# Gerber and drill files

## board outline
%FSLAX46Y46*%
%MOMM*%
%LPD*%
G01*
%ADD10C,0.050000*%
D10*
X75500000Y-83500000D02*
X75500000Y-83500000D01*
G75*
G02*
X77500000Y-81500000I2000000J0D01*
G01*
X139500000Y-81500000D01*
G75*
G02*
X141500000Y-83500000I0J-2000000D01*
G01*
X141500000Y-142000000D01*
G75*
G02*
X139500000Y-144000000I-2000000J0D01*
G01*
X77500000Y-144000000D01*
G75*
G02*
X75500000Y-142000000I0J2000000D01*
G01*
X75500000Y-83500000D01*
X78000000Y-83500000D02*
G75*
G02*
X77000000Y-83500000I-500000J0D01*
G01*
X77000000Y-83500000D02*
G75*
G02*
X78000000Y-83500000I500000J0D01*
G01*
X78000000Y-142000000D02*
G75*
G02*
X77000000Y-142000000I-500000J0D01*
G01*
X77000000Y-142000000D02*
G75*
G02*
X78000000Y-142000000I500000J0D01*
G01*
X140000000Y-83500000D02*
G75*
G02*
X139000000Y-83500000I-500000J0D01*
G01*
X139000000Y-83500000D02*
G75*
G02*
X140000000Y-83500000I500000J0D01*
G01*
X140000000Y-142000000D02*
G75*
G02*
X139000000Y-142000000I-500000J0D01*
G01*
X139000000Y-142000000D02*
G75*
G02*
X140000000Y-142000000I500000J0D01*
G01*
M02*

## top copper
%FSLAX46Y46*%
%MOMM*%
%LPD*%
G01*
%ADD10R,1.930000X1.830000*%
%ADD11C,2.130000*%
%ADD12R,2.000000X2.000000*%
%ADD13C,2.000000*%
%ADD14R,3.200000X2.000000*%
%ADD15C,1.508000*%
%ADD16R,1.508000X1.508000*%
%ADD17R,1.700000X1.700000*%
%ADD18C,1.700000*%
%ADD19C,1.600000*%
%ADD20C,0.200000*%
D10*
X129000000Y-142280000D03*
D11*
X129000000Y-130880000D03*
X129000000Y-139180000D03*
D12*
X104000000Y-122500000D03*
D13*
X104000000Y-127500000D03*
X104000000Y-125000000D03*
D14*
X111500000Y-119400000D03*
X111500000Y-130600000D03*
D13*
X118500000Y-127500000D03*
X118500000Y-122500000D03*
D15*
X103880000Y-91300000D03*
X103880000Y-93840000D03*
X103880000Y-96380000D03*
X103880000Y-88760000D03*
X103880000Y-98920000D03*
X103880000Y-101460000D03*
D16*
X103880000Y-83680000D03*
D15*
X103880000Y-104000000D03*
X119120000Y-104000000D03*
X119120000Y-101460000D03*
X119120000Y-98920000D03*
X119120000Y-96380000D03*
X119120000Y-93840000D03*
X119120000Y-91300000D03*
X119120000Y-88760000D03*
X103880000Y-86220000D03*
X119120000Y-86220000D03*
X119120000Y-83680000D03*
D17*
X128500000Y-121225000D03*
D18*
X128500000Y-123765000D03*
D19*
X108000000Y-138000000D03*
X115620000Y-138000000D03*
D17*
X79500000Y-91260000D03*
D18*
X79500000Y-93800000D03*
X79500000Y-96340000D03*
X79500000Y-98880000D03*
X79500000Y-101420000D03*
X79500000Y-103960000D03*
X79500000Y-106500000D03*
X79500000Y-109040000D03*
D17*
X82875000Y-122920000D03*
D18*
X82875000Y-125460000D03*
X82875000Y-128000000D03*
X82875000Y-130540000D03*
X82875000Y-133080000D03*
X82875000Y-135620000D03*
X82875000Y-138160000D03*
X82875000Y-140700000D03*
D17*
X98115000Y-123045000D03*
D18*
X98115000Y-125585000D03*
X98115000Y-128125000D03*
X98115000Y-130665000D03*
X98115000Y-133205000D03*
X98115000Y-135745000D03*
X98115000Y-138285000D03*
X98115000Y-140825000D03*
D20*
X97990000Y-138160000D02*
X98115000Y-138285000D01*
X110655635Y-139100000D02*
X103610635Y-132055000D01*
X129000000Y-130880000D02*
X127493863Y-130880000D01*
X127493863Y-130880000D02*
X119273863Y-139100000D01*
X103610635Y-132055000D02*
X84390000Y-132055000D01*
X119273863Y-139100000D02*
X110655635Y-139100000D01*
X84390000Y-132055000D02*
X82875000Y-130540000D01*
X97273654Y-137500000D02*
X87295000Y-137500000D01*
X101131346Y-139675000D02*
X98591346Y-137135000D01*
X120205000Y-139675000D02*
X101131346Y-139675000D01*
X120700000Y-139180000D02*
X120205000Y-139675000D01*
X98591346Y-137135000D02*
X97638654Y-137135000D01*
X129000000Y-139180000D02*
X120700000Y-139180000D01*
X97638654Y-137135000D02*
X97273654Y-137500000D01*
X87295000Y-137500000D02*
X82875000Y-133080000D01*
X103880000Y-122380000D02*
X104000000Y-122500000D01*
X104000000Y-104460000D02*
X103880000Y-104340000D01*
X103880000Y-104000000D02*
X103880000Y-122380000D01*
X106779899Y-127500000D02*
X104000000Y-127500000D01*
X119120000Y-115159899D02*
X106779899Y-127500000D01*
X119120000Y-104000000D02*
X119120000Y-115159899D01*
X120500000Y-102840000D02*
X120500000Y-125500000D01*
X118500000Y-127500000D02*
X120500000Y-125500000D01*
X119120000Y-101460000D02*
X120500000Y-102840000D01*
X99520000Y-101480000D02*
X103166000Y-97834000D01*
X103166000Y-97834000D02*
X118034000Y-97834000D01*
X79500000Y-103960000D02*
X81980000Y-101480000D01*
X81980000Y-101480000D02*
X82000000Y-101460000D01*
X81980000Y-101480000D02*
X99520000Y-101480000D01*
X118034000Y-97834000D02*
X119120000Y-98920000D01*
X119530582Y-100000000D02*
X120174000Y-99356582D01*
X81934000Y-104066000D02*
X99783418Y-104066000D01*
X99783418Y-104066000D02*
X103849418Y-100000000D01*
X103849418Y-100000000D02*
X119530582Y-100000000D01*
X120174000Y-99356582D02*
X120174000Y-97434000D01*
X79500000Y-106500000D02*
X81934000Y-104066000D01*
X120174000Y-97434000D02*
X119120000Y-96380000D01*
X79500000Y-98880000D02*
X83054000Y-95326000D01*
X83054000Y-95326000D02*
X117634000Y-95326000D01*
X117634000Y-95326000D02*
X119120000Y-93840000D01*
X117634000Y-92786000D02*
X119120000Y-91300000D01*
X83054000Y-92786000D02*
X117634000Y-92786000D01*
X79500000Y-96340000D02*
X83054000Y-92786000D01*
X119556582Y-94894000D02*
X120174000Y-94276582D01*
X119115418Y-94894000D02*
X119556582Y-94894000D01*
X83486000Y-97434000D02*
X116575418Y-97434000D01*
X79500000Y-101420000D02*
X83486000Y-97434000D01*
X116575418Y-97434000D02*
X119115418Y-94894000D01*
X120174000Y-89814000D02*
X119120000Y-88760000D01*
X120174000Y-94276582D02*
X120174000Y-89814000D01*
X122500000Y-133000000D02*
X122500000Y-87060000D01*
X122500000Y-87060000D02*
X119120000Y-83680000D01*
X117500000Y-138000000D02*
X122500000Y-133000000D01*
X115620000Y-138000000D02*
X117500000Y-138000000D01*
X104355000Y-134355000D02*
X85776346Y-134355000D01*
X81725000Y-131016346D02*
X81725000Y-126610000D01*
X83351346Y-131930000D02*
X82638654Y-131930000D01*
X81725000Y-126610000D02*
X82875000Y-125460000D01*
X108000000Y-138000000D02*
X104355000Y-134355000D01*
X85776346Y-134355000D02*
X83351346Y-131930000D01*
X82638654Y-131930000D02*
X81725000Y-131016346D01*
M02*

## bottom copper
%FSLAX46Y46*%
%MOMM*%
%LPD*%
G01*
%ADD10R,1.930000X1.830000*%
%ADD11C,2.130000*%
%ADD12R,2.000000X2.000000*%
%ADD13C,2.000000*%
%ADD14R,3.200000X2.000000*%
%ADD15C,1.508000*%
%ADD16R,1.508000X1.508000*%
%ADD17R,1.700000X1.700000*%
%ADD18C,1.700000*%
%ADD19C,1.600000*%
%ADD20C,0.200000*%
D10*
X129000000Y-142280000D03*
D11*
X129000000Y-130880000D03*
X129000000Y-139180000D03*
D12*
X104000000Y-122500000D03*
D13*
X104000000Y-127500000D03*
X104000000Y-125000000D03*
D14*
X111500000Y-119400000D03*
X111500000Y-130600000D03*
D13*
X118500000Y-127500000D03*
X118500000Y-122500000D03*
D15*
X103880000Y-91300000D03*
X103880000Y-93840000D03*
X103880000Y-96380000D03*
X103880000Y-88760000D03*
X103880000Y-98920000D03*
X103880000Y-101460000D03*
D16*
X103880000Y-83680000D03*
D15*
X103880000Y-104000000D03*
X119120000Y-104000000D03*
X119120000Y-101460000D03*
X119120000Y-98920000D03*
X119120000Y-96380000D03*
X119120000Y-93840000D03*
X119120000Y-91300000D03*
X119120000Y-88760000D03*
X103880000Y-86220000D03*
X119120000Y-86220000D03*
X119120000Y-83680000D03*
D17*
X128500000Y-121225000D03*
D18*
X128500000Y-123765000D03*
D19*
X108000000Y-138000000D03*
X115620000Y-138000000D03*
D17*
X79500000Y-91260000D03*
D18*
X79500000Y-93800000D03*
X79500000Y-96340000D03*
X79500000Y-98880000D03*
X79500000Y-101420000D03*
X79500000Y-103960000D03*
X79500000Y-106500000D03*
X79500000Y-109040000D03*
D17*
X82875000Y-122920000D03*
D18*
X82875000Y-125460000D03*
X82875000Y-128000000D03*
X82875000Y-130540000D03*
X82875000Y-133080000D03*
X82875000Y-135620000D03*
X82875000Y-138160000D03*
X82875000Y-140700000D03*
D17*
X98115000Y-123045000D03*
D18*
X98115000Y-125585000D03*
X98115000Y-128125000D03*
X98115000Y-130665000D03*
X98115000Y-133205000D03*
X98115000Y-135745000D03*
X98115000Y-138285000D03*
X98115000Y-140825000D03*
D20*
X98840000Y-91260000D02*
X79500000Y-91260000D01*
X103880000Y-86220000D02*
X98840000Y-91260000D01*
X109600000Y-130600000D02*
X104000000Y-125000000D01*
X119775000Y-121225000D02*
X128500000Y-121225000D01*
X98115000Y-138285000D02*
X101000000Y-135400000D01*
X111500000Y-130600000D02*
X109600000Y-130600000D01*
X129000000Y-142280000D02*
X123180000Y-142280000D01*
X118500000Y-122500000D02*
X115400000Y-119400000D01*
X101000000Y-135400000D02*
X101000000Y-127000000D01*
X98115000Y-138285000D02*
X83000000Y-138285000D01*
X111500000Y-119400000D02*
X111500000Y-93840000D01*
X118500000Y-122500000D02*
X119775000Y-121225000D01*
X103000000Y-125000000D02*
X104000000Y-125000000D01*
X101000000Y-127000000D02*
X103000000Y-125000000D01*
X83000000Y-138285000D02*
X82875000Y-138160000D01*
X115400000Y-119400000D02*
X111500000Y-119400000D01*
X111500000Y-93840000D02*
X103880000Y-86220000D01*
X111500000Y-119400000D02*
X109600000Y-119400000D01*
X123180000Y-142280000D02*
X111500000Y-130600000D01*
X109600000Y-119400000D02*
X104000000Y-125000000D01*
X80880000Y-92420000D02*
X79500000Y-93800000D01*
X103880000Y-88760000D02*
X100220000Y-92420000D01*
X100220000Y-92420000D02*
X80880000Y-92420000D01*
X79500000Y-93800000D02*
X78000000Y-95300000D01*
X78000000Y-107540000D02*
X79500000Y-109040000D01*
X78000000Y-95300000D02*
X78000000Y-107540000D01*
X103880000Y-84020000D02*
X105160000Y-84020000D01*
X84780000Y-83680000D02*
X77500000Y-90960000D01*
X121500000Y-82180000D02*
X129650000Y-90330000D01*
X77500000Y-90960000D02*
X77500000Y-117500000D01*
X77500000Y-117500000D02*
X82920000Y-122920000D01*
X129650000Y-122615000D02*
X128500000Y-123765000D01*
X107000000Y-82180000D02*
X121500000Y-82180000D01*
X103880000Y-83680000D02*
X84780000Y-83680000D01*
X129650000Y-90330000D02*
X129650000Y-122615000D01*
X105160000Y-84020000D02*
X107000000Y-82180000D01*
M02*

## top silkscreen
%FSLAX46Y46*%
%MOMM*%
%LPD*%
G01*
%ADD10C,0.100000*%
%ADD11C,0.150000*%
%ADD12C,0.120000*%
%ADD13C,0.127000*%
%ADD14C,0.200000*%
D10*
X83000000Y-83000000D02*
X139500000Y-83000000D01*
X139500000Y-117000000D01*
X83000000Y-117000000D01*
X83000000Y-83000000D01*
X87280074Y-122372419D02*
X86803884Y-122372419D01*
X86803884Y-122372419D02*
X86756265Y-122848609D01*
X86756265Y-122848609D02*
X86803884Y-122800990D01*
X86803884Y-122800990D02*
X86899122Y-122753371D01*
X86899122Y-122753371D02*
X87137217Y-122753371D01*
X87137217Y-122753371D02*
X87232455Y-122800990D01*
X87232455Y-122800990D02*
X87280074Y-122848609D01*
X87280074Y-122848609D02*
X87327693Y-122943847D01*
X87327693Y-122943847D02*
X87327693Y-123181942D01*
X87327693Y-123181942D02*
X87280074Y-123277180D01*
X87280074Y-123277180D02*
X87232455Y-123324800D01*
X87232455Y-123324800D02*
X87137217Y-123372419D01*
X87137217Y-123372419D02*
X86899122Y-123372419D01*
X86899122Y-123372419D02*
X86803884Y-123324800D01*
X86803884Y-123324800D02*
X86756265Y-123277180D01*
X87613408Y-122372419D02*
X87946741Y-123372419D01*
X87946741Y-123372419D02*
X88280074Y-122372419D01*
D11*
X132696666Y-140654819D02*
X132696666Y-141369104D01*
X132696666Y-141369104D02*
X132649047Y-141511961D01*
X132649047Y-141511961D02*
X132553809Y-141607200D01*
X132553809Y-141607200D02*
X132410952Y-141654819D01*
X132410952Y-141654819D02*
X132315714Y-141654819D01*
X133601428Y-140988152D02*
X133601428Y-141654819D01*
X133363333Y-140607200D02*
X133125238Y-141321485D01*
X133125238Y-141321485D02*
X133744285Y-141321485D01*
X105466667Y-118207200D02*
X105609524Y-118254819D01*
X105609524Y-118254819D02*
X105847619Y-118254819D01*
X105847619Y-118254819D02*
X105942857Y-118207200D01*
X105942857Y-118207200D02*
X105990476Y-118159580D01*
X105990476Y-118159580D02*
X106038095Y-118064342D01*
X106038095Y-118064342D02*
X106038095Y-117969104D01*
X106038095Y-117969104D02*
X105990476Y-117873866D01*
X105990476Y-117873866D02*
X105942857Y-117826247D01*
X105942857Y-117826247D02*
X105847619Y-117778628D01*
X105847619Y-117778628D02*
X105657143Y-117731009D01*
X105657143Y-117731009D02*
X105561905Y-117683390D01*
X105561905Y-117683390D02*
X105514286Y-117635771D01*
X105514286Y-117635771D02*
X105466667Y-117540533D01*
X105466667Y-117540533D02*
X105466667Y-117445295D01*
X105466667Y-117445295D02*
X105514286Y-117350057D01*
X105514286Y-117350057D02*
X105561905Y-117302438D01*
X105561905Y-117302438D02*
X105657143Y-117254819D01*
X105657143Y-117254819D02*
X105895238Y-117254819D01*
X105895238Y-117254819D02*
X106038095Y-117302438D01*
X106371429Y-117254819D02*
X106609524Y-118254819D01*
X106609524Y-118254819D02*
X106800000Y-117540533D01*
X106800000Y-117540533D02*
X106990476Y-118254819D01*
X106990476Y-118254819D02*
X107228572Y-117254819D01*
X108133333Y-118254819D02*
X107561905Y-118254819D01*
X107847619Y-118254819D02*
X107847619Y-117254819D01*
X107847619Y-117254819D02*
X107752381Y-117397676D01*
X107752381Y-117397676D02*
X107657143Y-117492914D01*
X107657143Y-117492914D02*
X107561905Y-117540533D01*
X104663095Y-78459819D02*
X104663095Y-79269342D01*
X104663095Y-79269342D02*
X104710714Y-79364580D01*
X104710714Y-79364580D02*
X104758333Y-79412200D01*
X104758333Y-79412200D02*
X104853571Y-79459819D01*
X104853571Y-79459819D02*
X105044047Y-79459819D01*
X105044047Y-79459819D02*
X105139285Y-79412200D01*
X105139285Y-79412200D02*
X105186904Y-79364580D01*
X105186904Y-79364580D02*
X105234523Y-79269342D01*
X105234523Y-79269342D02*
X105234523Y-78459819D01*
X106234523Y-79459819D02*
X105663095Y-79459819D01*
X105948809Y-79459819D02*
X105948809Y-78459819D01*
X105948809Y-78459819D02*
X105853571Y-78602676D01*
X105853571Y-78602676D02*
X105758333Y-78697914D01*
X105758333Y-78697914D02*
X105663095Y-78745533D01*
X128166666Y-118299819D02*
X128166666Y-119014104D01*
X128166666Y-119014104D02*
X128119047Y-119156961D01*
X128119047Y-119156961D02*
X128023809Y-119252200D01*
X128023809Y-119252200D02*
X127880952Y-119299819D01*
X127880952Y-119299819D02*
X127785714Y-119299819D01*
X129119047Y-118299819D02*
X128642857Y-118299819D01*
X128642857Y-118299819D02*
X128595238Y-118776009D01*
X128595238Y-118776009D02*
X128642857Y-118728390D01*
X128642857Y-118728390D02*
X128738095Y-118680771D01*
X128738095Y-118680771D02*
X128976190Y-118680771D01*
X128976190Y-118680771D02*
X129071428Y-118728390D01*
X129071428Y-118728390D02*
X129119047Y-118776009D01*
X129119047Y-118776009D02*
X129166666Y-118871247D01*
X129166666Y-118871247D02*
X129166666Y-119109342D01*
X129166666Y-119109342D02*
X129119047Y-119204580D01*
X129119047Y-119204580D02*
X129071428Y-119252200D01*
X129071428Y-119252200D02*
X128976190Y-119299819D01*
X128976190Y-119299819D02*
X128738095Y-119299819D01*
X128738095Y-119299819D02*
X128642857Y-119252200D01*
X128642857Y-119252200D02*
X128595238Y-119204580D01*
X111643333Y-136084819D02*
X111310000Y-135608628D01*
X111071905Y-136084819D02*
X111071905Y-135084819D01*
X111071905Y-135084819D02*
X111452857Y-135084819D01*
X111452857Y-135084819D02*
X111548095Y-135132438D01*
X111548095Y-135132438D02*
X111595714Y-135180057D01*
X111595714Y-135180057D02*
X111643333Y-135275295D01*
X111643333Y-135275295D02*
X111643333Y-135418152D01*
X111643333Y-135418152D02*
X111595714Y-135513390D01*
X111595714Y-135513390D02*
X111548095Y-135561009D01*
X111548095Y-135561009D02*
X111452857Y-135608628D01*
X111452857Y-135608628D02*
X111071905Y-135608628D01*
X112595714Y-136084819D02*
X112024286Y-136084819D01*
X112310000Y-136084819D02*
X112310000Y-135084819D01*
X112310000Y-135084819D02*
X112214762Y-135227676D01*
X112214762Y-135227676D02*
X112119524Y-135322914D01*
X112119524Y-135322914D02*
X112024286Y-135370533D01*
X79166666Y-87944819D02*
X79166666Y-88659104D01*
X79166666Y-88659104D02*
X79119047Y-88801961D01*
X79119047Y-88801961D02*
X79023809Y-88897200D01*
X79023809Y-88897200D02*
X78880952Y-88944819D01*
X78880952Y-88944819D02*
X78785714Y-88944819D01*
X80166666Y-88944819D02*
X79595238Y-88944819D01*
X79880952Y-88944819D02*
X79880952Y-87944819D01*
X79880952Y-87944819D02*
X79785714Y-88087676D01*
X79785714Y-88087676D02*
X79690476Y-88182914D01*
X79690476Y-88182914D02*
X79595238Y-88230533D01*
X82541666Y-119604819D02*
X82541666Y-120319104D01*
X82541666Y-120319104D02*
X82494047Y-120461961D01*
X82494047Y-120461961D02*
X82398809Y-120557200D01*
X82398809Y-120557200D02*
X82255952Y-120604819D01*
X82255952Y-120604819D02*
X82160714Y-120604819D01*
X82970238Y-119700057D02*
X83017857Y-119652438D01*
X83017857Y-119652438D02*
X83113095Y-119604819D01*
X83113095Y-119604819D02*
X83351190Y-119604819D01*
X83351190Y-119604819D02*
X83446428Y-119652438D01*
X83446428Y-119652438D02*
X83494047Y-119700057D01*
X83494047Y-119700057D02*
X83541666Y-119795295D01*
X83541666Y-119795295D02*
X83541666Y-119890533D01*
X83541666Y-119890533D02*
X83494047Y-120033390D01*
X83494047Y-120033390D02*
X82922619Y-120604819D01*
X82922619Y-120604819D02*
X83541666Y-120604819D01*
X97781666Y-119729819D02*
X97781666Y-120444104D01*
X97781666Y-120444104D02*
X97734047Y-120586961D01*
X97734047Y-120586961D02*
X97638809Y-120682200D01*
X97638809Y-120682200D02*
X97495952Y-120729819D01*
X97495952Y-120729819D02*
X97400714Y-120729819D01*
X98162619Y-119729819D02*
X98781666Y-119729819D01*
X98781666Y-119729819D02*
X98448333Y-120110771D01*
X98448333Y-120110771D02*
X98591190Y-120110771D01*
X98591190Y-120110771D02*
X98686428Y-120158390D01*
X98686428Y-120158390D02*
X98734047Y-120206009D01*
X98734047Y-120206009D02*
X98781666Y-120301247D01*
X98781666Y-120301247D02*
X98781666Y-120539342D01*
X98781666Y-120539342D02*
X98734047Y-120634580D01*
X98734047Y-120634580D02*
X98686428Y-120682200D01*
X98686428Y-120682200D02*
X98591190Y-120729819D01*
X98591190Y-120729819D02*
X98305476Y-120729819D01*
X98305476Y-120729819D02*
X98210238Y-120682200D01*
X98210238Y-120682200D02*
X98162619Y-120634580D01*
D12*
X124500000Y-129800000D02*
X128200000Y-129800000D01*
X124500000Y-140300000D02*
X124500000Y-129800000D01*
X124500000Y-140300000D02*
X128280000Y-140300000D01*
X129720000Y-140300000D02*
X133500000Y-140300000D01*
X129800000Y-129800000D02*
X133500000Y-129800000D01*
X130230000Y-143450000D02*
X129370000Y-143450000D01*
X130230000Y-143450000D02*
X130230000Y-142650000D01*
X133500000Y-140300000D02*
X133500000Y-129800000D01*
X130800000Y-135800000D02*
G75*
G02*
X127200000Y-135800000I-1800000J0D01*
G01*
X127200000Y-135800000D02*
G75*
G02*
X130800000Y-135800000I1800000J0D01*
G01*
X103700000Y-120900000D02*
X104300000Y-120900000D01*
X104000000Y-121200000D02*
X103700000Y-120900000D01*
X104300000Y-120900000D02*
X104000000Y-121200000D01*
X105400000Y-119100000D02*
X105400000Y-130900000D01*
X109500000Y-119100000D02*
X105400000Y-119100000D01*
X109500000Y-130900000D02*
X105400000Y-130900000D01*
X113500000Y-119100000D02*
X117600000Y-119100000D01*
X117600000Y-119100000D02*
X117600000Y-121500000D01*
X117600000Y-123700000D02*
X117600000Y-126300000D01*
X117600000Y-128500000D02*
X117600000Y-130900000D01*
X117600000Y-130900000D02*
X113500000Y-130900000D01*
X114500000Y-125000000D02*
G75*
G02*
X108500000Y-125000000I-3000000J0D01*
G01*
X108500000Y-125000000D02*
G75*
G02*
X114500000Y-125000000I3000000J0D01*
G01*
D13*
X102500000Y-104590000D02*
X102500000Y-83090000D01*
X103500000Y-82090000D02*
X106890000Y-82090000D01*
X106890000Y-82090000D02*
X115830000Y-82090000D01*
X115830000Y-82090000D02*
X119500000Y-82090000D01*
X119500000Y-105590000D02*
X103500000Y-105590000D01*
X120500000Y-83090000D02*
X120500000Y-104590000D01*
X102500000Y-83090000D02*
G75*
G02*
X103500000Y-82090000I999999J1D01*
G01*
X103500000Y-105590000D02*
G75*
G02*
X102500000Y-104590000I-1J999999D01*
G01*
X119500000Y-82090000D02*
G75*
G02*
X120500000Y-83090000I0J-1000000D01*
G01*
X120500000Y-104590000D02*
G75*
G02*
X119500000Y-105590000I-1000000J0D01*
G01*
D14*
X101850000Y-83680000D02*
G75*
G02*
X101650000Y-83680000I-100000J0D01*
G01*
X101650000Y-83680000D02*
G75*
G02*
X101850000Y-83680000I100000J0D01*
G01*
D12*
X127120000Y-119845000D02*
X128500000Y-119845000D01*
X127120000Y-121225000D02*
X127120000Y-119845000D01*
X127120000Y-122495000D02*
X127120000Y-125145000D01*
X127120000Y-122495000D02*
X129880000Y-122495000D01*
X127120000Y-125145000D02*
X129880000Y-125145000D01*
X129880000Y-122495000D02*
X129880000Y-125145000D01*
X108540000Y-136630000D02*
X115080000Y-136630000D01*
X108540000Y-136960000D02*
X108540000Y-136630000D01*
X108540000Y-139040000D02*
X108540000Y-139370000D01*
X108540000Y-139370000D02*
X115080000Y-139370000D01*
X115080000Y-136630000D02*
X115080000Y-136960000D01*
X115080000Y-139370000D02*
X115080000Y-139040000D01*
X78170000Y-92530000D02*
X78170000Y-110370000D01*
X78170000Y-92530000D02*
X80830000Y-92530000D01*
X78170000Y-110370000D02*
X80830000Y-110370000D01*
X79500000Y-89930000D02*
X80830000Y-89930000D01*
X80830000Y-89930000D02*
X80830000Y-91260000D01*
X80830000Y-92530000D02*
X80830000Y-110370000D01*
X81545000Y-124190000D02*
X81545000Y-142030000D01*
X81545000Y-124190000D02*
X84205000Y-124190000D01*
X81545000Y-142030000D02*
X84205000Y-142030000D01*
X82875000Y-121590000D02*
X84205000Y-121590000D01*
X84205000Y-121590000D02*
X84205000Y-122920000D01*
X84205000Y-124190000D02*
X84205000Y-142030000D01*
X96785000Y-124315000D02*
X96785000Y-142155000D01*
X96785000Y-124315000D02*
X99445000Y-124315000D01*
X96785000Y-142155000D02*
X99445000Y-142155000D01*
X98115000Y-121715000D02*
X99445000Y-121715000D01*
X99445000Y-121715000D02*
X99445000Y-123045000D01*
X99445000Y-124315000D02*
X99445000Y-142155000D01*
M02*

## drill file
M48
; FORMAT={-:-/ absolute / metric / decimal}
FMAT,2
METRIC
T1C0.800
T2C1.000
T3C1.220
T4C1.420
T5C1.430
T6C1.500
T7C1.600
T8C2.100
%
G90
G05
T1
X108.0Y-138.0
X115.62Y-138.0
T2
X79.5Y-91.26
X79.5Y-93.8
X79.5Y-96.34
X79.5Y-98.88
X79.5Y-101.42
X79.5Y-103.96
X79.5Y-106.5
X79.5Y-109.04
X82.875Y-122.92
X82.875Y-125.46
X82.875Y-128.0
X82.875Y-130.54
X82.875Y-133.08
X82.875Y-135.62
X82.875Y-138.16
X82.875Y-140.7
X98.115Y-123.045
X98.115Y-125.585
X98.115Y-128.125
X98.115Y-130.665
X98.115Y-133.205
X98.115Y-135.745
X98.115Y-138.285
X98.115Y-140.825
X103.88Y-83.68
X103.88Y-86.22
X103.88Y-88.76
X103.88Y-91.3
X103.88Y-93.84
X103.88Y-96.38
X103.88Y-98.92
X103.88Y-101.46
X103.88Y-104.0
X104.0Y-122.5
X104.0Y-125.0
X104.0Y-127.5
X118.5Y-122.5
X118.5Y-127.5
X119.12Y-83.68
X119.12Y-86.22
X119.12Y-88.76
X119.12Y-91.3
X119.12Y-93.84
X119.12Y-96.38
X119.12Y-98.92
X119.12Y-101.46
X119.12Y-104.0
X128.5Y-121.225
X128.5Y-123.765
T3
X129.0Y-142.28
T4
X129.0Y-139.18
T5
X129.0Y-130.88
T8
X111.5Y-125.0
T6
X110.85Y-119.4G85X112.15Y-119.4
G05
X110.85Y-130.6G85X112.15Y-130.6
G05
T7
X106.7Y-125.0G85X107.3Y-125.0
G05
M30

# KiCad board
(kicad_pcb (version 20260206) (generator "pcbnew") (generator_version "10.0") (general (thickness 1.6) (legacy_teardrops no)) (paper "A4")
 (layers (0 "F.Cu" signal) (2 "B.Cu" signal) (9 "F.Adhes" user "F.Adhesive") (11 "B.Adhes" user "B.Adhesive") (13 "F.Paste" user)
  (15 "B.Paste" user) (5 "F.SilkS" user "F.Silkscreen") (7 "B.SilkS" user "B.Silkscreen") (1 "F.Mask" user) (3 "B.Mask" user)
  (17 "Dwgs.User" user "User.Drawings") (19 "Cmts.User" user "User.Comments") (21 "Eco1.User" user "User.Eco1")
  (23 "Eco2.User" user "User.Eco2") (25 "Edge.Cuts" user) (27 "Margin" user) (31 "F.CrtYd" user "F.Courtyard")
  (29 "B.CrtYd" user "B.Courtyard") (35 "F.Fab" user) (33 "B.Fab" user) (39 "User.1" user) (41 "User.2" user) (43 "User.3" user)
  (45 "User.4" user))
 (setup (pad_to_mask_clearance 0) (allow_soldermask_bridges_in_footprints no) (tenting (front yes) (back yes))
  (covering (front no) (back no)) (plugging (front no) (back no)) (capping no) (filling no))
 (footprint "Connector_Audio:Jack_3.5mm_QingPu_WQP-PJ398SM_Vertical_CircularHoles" (layer "F.Cu") (at 129 142.28 180)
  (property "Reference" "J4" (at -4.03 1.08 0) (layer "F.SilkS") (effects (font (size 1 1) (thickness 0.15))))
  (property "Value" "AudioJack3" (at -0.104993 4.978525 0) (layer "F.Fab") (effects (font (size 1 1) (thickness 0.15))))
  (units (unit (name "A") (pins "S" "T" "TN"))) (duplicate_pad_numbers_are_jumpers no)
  (fp_line (start 4.5 12.48) (end 0.8 12.48) (stroke (width 0.12) (type solid)) (layer "F.SilkS"))
  (fp_line (start 4.5 1.98) (end 4.5 12.48) (stroke (width 0.12) (type solid)) (layer "F.SilkS"))
  (fp_line (start 4.5 1.98) (end 0.72 1.98) (stroke (width 0.12) (type solid)) (layer "F.SilkS"))
  (fp_line (start -0.72 1.98) (end -4.5 1.98) (stroke (width 0.12) (type solid)) (layer "F.SilkS"))
  (fp_line (start -0.8 12.48) (end -4.5 12.48) (stroke (width 0.12) (type solid)) (layer "F.SilkS"))
  (fp_line (start -1.23 -1.17) (end -0.37 -1.17) (stroke (width 0.12) (type solid)) (layer "F.SilkS"))
  (fp_line (start -1.23 -1.17) (end -1.23 -0.37) (stroke (width 0.12) (type solid)) (layer "F.SilkS"))
  (fp_line (start -4.5 1.98) (end -4.5 12.48) (stroke (width 0.12) (type solid)) (layer "F.SilkS"))
  (fp_circle (center 0 6.48) (end 1.8 6.48) (stroke (width 0.12) (type solid)) (fill no) (layer "F.SilkS"))
  (pad "S" thru_hole rect (at 0 0) (size 1.93 1.83) (drill 1.22) (layers "*.Cu" "*.Mask") (remove_unused_layers no) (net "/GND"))
  (pad "T" thru_hole circle (at 0 11.4) (size 2.13 2.13) (drill 1.43) (layers "*.Cu" "*.Mask") (remove_unused_layers no) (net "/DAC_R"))
  (pad "TN" thru_hole circle (at 0 3.1) (size 2.13 2.13) (drill 1.42) (layers "*.Cu" "*.Mask") (remove_unused_layers no) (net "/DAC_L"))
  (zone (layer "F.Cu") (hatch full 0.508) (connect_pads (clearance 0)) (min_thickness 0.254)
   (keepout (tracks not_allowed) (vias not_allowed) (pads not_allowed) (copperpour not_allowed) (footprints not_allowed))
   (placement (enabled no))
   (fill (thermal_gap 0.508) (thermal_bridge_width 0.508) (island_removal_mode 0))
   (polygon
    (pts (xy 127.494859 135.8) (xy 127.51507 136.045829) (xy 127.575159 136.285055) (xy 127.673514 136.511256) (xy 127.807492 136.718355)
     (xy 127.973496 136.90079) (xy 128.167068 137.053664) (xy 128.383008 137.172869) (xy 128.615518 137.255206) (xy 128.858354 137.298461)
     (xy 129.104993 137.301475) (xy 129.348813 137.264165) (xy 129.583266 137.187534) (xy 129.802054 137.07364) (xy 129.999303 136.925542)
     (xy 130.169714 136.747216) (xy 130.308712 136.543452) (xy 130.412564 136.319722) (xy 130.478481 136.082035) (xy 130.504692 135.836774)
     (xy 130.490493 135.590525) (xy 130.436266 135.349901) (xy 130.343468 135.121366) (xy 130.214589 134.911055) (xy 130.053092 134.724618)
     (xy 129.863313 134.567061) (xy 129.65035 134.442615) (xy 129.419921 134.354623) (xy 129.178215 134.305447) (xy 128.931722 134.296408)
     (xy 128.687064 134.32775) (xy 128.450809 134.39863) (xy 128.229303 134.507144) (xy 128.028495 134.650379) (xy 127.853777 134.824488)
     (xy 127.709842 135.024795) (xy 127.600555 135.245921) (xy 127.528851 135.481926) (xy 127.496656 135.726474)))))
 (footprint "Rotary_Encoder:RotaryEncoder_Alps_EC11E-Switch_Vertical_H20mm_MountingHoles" (layer "F.Cu") (at 104 122.5)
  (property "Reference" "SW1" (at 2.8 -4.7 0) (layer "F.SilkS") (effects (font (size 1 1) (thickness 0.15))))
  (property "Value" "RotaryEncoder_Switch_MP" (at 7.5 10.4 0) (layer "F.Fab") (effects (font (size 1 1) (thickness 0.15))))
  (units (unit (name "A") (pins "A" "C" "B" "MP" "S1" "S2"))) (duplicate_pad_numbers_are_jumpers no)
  (fp_line (start -0.3 -1.6) (end 0.3 -1.6) (stroke (width 0.12) (type solid)) (layer "F.SilkS"))
  (fp_line (start 0 -1.3) (end -0.3 -1.6) (stroke (width 0.12) (type solid)) (layer "F.SilkS"))
  (fp_line (start 0.3 -1.6) (end 0 -1.3) (stroke (width 0.12) (type solid)) (layer "F.SilkS"))
  (fp_line (start 1.4 -3.4) (end 1.4 8.4) (stroke (width 0.12) (type solid)) (layer "F.SilkS"))
  (fp_line (start 5.5 -3.4) (end 1.4 -3.4) (stroke (width 0.12) (type solid)) (layer "F.SilkS"))
  (fp_line (start 5.5 8.4) (end 1.4 8.4) (stroke (width 0.12) (type solid)) (layer "F.SilkS"))
  (fp_line (start 9.5 -3.4) (end 13.6 -3.4) (stroke (width 0.12) (type solid)) (layer "F.SilkS"))
  (fp_line (start 13.6 -3.4) (end 13.6 -1) (stroke (width 0.12) (type solid)) (layer "F.SilkS"))
  (fp_line (start 13.6 1.2) (end 13.6 3.8) (stroke (width 0.12) (type solid)) (layer "F.SilkS"))
  (fp_line (start 13.6 6) (end 13.6 8.4) (stroke (width 0.12) (type solid)) (layer "F.SilkS"))
  (fp_line (start 13.6 8.4) (end 9.5 8.4) (stroke (width 0.12) (type solid)) (layer "F.SilkS"))
  (fp_circle (center 7.5 2.5) (end 10.5 2.5) (stroke (width 0.12) (type solid)) (fill no) (layer "F.SilkS"))
  (pad "" np_thru_hole oval (at 3 2.5) (size 2.2 1.6) (drill oval 2.2 1.6) (layers "*.Mask"))
  (pad "" np_thru_hole circle (at 7.5 2.5) (size 2.1 2.1) (drill 2.1) (layers "*.Mask"))
  (pad "A" thru_hole rect (at 0 0) (size 2 2) (drill 1) (layers "*.Cu" "*.Mask") (remove_unused_layers no) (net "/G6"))
  (pad "B" thru_hole circle (at 0 5) (size 2 2) (drill 1) (layers "*.Cu" "*.Mask") (remove_unused_layers no) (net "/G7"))
  (pad "C" thru_hole circle (at 0 2.5) (size 2 2) (drill 1) (layers "*.Cu" "*.Mask") (remove_unused_layers no) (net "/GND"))
  (pad "MP" thru_hole rect (at 7.5 -3.1) (size 3.2 2) (drill oval 2.8 1.5) (layers "*.Cu" "*.Mask") (remove_unused_layers no) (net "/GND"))
  (pad "MP" thru_hole rect (at 7.5 8.1) (size 3.2 2) (drill oval 2.8 1.5) (layers "*.Cu" "*.Mask") (remove_unused_layers no) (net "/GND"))
  (pad "S1" thru_hole circle (at 14.5 5) (size 2 2) (drill 1) (layers "*.Cu" "*.Mask") (remove_unused_layers no) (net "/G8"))
  (pad "S2" thru_hole circle (at 14.5 0) (size 2 2) (drill 1) (layers "*.Cu" "*.Mask") (remove_unused_layers no) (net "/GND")))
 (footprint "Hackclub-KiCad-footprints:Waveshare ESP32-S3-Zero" (layer "F.Cu") (at 111.5 93.84)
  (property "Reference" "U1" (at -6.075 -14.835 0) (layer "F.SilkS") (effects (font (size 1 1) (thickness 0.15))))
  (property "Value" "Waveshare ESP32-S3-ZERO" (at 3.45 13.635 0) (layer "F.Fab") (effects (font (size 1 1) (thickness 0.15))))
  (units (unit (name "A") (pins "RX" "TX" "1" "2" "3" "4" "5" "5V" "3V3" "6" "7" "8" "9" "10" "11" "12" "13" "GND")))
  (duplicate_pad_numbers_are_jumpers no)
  (fp_line (start -9 10.75) (end -9 -10.75) (stroke (width 0.127) (type solid)) (layer "F.SilkS"))
  (fp_line (start -8 -11.75) (end -4.61 -11.75) (stroke (width 0.127) (type solid)) (layer "F.SilkS"))
  (fp_line (start -4.61 -11.75) (end 4.33 -11.75) (stroke (width 0.127) (type solid)) (layer "F.SilkS"))
  (fp_line (start 4.33 -11.75) (end 8 -11.75) (stroke (width 0.127) (type solid)) (layer "F.SilkS"))
  (fp_line (start 8 11.75) (end -8 11.75) (stroke (width 0.127) (type solid)) (layer "F.SilkS"))
  (fp_line (start 9 -10.75) (end 9 10.75) (stroke (width 0.127) (type solid)) (layer "F.SilkS"))
  (fp_arc (start -9 -10.75) (mid -8.707107 -11.457107) (end -8 -11.75) (stroke (width 0.127) (type solid)) (layer "F.SilkS"))
  (fp_arc (start -8 11.75) (mid -8.707107 11.457107) (end -9 10.75) (stroke (width 0.127) (type solid)) (layer "F.SilkS"))
  (fp_arc (start 8 -11.75) (mid 8.707107 -11.457107) (end 9 -10.75) (stroke (width 0.127) (type solid)) (layer "F.SilkS"))
  (fp_arc (start 9 10.75) (mid 8.707107 11.457107) (end 8 11.75) (stroke (width 0.127) (type solid)) (layer "F.SilkS"))
  (fp_circle (center -9.75 -10.16) (end -9.65 -10.16) (stroke (width 0.2) (type solid)) (fill no) (layer "F.SilkS"))
  (pad "1" thru_hole circle (at -7.62 -2.54) (size 1.508 1.508) (drill 1) (layers "*.Cu" "*.Mask") (remove_unused_layers no)
   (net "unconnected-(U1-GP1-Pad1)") (solder_mask_margin 0.102))
  (pad "2" thru_hole circle (at -7.62 0) (size 1.508 1.508) (drill 1) (layers "*.Cu" "*.Mask") (remove_unused_layers no)
   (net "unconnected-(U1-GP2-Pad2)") (solder_mask_margin 0.102))
  (pad "3" thru_hole circle (at -7.62 2.54) (size 1.508 1.508) (drill 1) (layers "*.Cu" "*.Mask") (remove_unused_layers no)
   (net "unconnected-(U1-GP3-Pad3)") (solder_mask_margin 0.102))
  (pad "3V3" thru_hole circle (at -7.62 -5.08) (size 1.508 1.508) (drill 1) (layers "*.Cu" "*.Mask") (remove_unused_layers no) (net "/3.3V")
   (solder_mask_margin 0.102))
  (pad "4" thru_hole circle (at -7.62 5.08) (size 1.508 1.508) (drill 1) (layers "*.Cu" "*.Mask") (remove_unused_layers no)
   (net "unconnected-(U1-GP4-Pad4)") (solder_mask_margin 0.102))
  (pad "5" thru_hole circle (at -7.62 7.62) (size 1.508 1.508) (drill 1) (layers "*.Cu" "*.Mask") (remove_unused_layers no)
   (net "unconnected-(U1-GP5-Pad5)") (solder_mask_margin 0.102))
  (pad "5V" thru_hole rect (at -7.62 -10.16) (size 1.508 1.508) (drill 1) (layers "*.Cu" "*.Mask") (remove_unused_layers no) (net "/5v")
   (solder_mask_margin 0.102))
  (pad "6" thru_hole circle (at -7.62 10.16) (size 1.508 1.508) (drill 1) (layers "*.Cu" "*.Mask") (remove_unused_layers no) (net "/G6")
   (solder_mask_margin 0.102))
  (pad "7" thru_hole circle (at 7.62 10.16) (size 1.508 1.508) (drill 1) (layers "*.Cu" "*.Mask") (remove_unused_layers no) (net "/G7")
   (solder_mask_margin 0.102))
  (pad "8" thru_hole circle (at 7.62 7.62) (size 1.508 1.508) (drill 1) (layers "*.Cu" "*.Mask") (remove_unused_layers no) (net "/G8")
   (solder_mask_margin 0.102))
  (pad "9" thru_hole circle (at 7.62 5.08) (size 1.508 1.508) (drill 1) (layers "*.Cu" "*.Mask") (remove_unused_layers no)
   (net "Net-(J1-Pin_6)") (solder_mask_margin 0.102))
  (pad "10" thru_hole circle (at 7.62 2.54) (size 1.508 1.508) (drill 1) (layers "*.Cu" "*.Mask") (remove_unused_layers no)
   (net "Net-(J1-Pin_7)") (solder_mask_margin 0.102))
  (pad "11" thru_hole circle (at 7.62 0) (size 1.508 1.508) (drill 1) (layers "*.Cu" "*.Mask") (remove_unused_layers no)
   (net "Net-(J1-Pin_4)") (solder_mask_margin 0.102))
  (pad "12" thru_hole circle (at 7.62 -2.54) (size 1.508 1.508) (drill 1) (layers "*.Cu" "*.Mask") (remove_unused_layers no)
   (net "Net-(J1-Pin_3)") (solder_mask_margin 0.102))
  (pad "13" thru_hole circle (at 7.62 -5.08) (size 1.508 1.508) (drill 1) (layers "*.Cu" "*.Mask") (remove_unused_layers no)
   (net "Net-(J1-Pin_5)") (solder_mask_margin 0.102))
  (pad "GND" thru_hole circle (at -7.62 -7.62) (size 1.508 1.508) (drill 1) (layers "*.Cu" "*.Mask") (remove_unused_layers no) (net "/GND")
   (solder_mask_margin 0.102))
  (pad "RX" thru_hole circle (at 7.62 -7.62) (size 1.508 1.508) (drill 1) (layers "*.Cu" "*.Mask") (remove_unused_layers no)
   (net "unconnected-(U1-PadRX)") (solder_mask_margin 0.102))
  (pad "TX" thru_hole circle (at 7.62 -10.16) (size 1.508 1.508) (drill 1) (layers "*.Cu" "*.Mask") (remove_unused_layers no)
   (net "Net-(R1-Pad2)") (solder_mask_margin 0.102)))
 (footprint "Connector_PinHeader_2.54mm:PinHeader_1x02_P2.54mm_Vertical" (layer "F.Cu") (at 128.5 121.225)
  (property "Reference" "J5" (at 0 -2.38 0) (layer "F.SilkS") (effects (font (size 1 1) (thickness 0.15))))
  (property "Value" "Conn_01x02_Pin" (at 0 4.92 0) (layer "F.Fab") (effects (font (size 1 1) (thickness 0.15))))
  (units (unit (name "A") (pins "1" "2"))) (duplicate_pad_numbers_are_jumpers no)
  (fp_line (start -1.38 -1.38) (end 0 -1.38) (stroke (width 0.12) (type solid)) (layer "F.SilkS"))
  (fp_line (start -1.38 0) (end -1.38 -1.38) (stroke (width 0.12) (type solid)) (layer "F.SilkS"))
  (fp_line (start -1.38 1.27) (end -1.38 3.92) (stroke (width 0.12) (type solid)) (layer "F.SilkS"))
  (fp_line (start -1.38 1.27) (end 1.38 1.27) (stroke (width 0.12) (type solid)) (layer "F.SilkS"))
  (fp_line (start -1.38 3.92) (end 1.38 3.92) (stroke (width 0.12) (type solid)) (layer "F.SilkS"))
  (fp_line (start 1.38 1.27) (end 1.38 3.92) (stroke (width 0.12) (type solid)) (layer "F.SilkS"))
  (pad "1" thru_hole rect (at 0 0) (size 1.7 1.7) (drill 1) (layers "*.Cu" "*.Mask") (remove_unused_layers no) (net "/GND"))
  (pad "2" thru_hole circle (at 0 2.54) (size 1.7 1.7) (drill 1) (layers "*.Cu" "*.Mask") (remove_unused_layers no) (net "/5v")))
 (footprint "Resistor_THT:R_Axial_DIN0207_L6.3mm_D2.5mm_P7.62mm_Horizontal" (layer "F.Cu") (at 108 138)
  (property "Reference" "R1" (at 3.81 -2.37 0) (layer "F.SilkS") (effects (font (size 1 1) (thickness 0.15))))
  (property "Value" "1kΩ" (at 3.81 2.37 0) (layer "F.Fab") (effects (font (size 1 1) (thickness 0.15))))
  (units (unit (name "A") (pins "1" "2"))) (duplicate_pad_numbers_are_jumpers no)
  (fp_line (start 0.54 -1.37) (end 7.08 -1.37) (stroke (width 0.12) (type solid)) (layer "F.SilkS"))
  (fp_line (start 0.54 -1.04) (end 0.54 -1.37) (stroke (width 0.12) (type solid)) (layer "F.SilkS"))
  (fp_line (start 0.54 1.04) (end 0.54 1.37) (stroke (width 0.12) (type solid)) (layer "F.SilkS"))
  (fp_line (start 0.54 1.37) (end 7.08 1.37) (stroke (width 0.12) (type solid)) (layer "F.SilkS"))
  (fp_line (start 7.08 -1.37) (end 7.08 -1.04) (stroke (width 0.12) (type solid)) (layer "F.SilkS"))
  (fp_line (start 7.08 1.37) (end 7.08 1.04) (stroke (width 0.12) (type solid)) (layer "F.SilkS"))
  (pad "1" thru_hole circle (at 0 0) (size 1.6 1.6) (drill 0.8) (layers "*.Cu" "*.Mask") (remove_unused_layers no) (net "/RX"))
  (pad "2" thru_hole circle (at 7.62 0) (size 1.6 1.6) (drill 0.8) (layers "*.Cu" "*.Mask") (remove_unused_layers no) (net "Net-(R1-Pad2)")))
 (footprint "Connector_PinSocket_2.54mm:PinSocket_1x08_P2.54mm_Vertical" (layer "F.Cu") (at 79.5 91.26)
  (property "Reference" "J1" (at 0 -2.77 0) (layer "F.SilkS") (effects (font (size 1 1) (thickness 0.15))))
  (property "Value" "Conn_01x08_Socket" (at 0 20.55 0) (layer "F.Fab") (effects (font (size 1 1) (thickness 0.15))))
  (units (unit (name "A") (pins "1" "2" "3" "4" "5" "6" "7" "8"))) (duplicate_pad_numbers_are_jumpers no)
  (fp_line (start -1.33 1.27) (end -1.33 19.11) (stroke (width 0.12) (type solid)) (layer "F.SilkS"))
  (fp_line (start -1.33 1.27) (end 1.33 1.27) (stroke (width 0.12) (type solid)) (layer "F.SilkS"))
  (fp_line (start -1.33 19.11) (end 1.33 19.11) (stroke (width 0.12) (type solid)) (layer "F.SilkS"))
  (fp_line (start 0 -1.33) (end 1.33 -1.33) (stroke (width 0.12) (type solid)) (layer "F.SilkS"))
  (fp_line (start 1.33 -1.33) (end 1.33 0) (stroke (width 0.12) (type solid)) (layer "F.SilkS"))
  (fp_line (start 1.33 1.27) (end 1.33 19.11) (stroke (width 0.12) (type solid)) (layer "F.SilkS"))
  (pad "1" thru_hole rect (at 0 0) (size 1.7 1.7) (drill 1) (layers "*.Cu" "*.Mask") (remove_unused_layers no) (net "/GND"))
  (pad "2" thru_hole circle (at 0 2.54) (size 1.7 1.7) (drill 1) (layers "*.Cu" "*.Mask") (remove_unused_layers no) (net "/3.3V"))
  (pad "3" thru_hole circle (at 0 5.08) (size 1.7 1.7) (drill 1) (layers "*.Cu" "*.Mask") (remove_unused_layers no) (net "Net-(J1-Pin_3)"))
  (pad "4" thru_hole circle (at 0 7.62) (size 1.7 1.7) (drill 1) (layers "*.Cu" "*.Mask") (remove_unused_layers no) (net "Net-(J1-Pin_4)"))
  (pad "5" thru_hole circle (at 0 10.16) (size 1.7 1.7) (drill 1) (layers "*.Cu" "*.Mask") (remove_unused_layers no) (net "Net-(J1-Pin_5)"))
  (pad "6" thru_hole circle (at 0 12.7) (size 1.7 1.7) (drill 1) (layers "*.Cu" "*.Mask") (remove_unused_layers no) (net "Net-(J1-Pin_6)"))
  (pad "7" thru_hole circle (at 0 15.24) (size 1.7 1.7) (drill 1) (layers "*.Cu" "*.Mask") (remove_unused_layers no) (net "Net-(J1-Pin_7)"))
  (pad "8" thru_hole circle (at 0 17.78) (size 1.7 1.7) (drill 1) (layers "*.Cu" "*.Mask") (remove_unused_layers no) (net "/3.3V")))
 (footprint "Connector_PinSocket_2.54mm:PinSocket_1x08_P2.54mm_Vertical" (layer "F.Cu") (at 82.875 122.92)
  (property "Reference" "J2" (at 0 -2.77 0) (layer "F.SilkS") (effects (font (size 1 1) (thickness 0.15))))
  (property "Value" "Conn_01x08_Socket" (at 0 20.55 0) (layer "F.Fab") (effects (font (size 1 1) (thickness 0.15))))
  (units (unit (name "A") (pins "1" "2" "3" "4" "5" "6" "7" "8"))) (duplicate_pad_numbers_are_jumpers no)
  (fp_line (start -1.33 1.27) (end -1.33 19.11) (stroke (width 0.12) (type solid)) (layer "F.SilkS"))
  (fp_line (start -1.33 1.27) (end 1.33 1.27) (stroke (width 0.12) (type solid)) (layer "F.SilkS"))
  (fp_line (start -1.33 19.11) (end 1.33 19.11) (stroke (width 0.12) (type solid)) (layer "F.SilkS"))
  (fp_line (start 0 -1.33) (end 1.33 -1.33) (stroke (width 0.12) (type solid)) (layer "F.SilkS"))
  (fp_line (start 1.33 -1.33) (end 1.33 0) (stroke (width 0.12) (type solid)) (layer "F.SilkS"))
  (fp_line (start 1.33 1.27) (end 1.33 19.11) (stroke (width 0.12) (type solid)) (layer "F.SilkS"))
  (pad "1" thru_hole rect (at 0 0) (size 1.7 1.7) (drill 1) (layers "*.Cu" "*.Mask") (remove_unused_layers no) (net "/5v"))
  (pad "2" thru_hole circle (at 0 2.54) (size 1.7 1.7) (drill 1) (layers "*.Cu" "*.Mask") (remove_unused_layers no) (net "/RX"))
  (pad "3" thru_hole circle (at 0 5.08) (size 1.7 1.7) (drill 1) (layers "*.Cu" "*.Mask") (remove_unused_layers no)
   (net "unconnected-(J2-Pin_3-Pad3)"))
  (pad "4" thru_hole circle (at 0 7.62) (size 1.7 1.7) (drill 1) (layers "*.Cu" "*.Mask") (remove_unused_layers no) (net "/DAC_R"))
  (pad "5" thru_hole circle (at 0 10.16) (size 1.7 1.7) (drill 1) (layers "*.Cu" "*.Mask") (remove_unused_layers no) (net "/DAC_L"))
  (pad "6" thru_hole circle (at 0 12.7) (size 1.7 1.7) (drill 1) (layers "*.Cu" "*.Mask") (remove_unused_layers no)
   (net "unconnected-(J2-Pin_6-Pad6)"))
  (pad "7" thru_hole circle (at 0 15.24) (size 1.7 1.7) (drill 1) (layers "*.Cu" "*.Mask") (remove_unused_layers no) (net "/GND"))
  (pad "8" thru_hole circle (at 0 17.78) (size 1.7 1.7) (drill 1) (layers "*.Cu" "*.Mask") (remove_unused_layers no)
   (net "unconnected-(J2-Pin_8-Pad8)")))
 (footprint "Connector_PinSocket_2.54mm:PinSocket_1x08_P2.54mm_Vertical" (layer "F.Cu") (at 98.115 123.045)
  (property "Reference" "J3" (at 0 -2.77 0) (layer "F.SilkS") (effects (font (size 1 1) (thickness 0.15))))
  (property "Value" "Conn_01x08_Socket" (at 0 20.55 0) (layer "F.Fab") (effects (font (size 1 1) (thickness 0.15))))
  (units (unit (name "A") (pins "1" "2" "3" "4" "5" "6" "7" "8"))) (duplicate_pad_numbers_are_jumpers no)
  (fp_line (start -1.33 1.27) (end -1.33 19.11) (stroke (width 0.12) (type solid)) (layer "F.SilkS"))
  (fp_line (start -1.33 1.27) (end 1.33 1.27) (stroke (width 0.12) (type solid)) (layer "F.SilkS"))
  (fp_line (start -1.33 19.11) (end 1.33 19.11) (stroke (width 0.12) (type solid)) (layer "F.SilkS"))
  (fp_line (start 0 -1.33) (end 1.33 -1.33) (stroke (width 0.12) (type solid)) (layer "F.SilkS"))
  (fp_line (start 1.33 -1.33) (end 1.33 0) (stroke (width 0.12) (type solid)) (layer "F.SilkS"))
  (fp_line (start 1.33 1.27) (end 1.33 19.11) (stroke (width 0.12) (type solid)) (layer "F.SilkS"))
  (pad "1" thru_hole rect (at 0 0) (size 1.7 1.7) (drill 1) (layers "*.Cu" "*.Mask") (remove_unused_layers no)
   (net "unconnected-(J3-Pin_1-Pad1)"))
  (pad "2" thru_hole circle (at 0 2.54) (size 1.7 1.7) (drill 1) (layers "*.Cu" "*.Mask") (remove_unused_layers no)
   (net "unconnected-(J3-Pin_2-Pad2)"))
  (pad "3" thru_hole circle (at 0 5.08) (size 1.7 1.7) (drill 1) (layers "*.Cu" "*.Mask") (remove_unused_layers no)
   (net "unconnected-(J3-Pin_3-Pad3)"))
  (pad "4" thru_hole circle (at 0 7.62) (size 1.7 1.7) (drill 1) (layers "*.Cu" "*.Mask") (remove_unused_layers no)
   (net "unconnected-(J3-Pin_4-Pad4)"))
  (pad "5" thru_hole circle (at 0 10.16) (size 1.7 1.7) (drill 1) (layers "*.Cu" "*.Mask") (remove_unused_layers no)
   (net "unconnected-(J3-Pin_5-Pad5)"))
  (pad "6" thru_hole circle (at 0 12.7) (size 1.7 1.7) (drill 1) (layers "*.Cu" "*.Mask") (remove_unused_layers no)
   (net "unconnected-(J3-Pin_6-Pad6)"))
  (pad "7" thru_hole circle (at 0 15.24) (size 1.7 1.7) (drill 1) (layers "*.Cu" "*.Mask") (remove_unused_layers no) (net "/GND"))
  (pad "8" thru_hole circle (at 0 17.78) (size 1.7 1.7) (drill 1) (layers "*.Cu" "*.Mask") (remove_unused_layers no)
   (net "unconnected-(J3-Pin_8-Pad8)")))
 (gr_rect (start 83 83) (end 139.5 117) (stroke (width 0.1) (type default)) (fill no) (layer "F.SilkS"))
 (gr_rect (start 75.5 81.5) (end 141.5 144) (radius 2) (stroke (width 0.05) (type solid)) (fill no) (layer "Edge.Cuts"))
 (gr_circle (center 77.5 83.5) (end 77.5 83) (stroke (width 0.05) (type default)) (fill no) (layer "Edge.Cuts"))
 (gr_circle (center 77.5 142) (end 78 142) (stroke (width 0.05) (type default)) (fill no) (layer "Edge.Cuts"))
 (gr_circle (center 139.5 83.5) (end 139.5 83) (stroke (width 0.05) (type default)) (fill no) (layer "Edge.Cuts"))
 (gr_circle (center 139.5 142) (end 139.5 141.5) (stroke (width 0.05) (type default)) (fill no) (layer "Edge.Cuts"))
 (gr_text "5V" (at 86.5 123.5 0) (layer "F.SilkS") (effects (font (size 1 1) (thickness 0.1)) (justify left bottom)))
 (segment (start 97.99 138.16) (end 98.115 138.285) (width 0.2) (layer "F.Cu") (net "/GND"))
 (segment (start 98.84 91.26) (end 79.5 91.26) (width 0.2) (layer "B.Cu") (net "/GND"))
 (segment (start 103.88 86.22) (end 98.84 91.26) (width 0.2) (layer "B.Cu") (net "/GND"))
 (segment (start 109.6 130.6) (end 104 125) (width 0.2) (layer "B.Cu") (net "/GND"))
 (segment (start 119.775 121.225) (end 128.5 121.225) (width 0.2) (layer "B.Cu") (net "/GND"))
 (segment (start 98.115 138.285) (end 101 135.4) (width 0.2) (layer "B.Cu") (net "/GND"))
 (segment (start 111.5 130.6) (end 109.6 130.6) (width 0.2) (layer "B.Cu") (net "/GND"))
 (segment (start 129 142.28) (end 123.18 142.28) (width 0.2) (layer "B.Cu") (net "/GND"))
 (segment (start 118.5 122.5) (end 115.4 119.4) (width 0.2) (layer "B.Cu") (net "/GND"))
 (segment (start 101 135.4) (end 101 127) (width 0.2) (layer "B.Cu") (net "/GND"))
 (segment (start 98.115 138.285) (end 83 138.285) (width 0.2) (layer "B.Cu") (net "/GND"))
 (segment (start 111.5 119.4) (end 111.5 93.84) (width 0.2) (layer "B.Cu") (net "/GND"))
 (segment (start 118.5 122.5) (end 119.775 121.225) (width 0.2) (layer "B.Cu") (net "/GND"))
 (segment (start 103 125) (end 104 125) (width 0.2) (layer "B.Cu") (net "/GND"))
 (segment (start 101 127) (end 103 125) (width 0.2) (layer "B.Cu") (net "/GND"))
 (segment (start 83 138.285) (end 82.875 138.16) (width 0.2) (layer "B.Cu") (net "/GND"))
 (segment (start 115.4 119.4) (end 111.5 119.4) (width 0.2) (layer "B.Cu") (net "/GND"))
 (segment (start 111.5 93.84) (end 103.88 86.22) (width 0.2) (layer "B.Cu") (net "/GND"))
 (segment (start 111.5 119.4) (end 109.6 119.4) (width 0.2) (layer "B.Cu") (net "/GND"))
 (segment (start 123.18 142.28) (end 111.5 130.6) (width 0.2) (layer "B.Cu") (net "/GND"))
 (segment (start 109.6 119.4) (end 104 125) (width 0.2) (layer "B.Cu") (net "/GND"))
 (segment (start 110.655635 139.1) (end 103.610635 132.055) (width 0.2) (layer "F.Cu") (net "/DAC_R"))
 (segment (start 129 130.88) (end 127.493863 130.88) (width 0.2) (layer "F.Cu") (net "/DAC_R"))
 (segment (start 127.493863 130.88) (end 119.273863 139.1) (width 0.2) (layer "F.Cu") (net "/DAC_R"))
 (segment (start 103.610635 132.055) (end 84.39 132.055) (width 0.2) (layer "F.Cu") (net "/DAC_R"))
 (segment (start 119.273863 139.1) (end 110.655635 139.1) (width 0.2) (layer "F.Cu") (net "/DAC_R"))
 (segment (start 84.39 132.055) (end 82.875 130.54) (width 0.2) (layer "F.Cu") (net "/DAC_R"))
 (segment (start 97.273654 137.5) (end 87.295 137.5) (width 0.2) (layer "F.Cu") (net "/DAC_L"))
 (segment (start 101.131346 139.675) (end 98.591346 137.135) (width 0.2) (layer "F.Cu") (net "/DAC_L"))
 (segment (start 120.205 139.675) (end 101.131346 139.675) (width 0.2) (layer "F.Cu") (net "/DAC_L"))
 (segment (start 120.7 139.18) (end 120.205 139.675) (width 0.2) (layer "F.Cu") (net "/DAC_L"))
 (segment (start 98.591346 137.135) (end 97.638654 137.135) (width 0.2) (layer "F.Cu") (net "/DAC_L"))
 (segment (start 129 139.18) (end 120.7 139.18) (width 0.2) (layer "F.Cu") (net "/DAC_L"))
 (segment (start 97.638654 137.135) (end 97.273654 137.5) (width 0.2) (layer "F.Cu") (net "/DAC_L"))
 (segment (start 87.295 137.5) (end 82.875 133.08) (width 0.2) (layer "F.Cu") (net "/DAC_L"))
 (segment (start 103.88 122.38) (end 104 122.5) (width 0.2) (layer "F.Cu") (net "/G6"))
 (segment (start 104 104.46) (end 103.88 104.34) (width 0.2) (layer "F.Cu") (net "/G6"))
 (segment (start 103.88 104) (end 103.88 122.38) (width 0.2) (layer "F.Cu") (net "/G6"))
 (segment (start 106.779899 127.5) (end 104 127.5) (width 0.2) (layer "F.Cu") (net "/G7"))
 (segment (start 119.12 115.159899) (end 106.779899 127.5) (width 0.2) (layer "F.Cu") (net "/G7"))
 (segment (start 119.12 104) (end 119.12 115.159899) (width 0.2) (layer "F.Cu") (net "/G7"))
 (segment (start 120.5 102.84) (end 120.5 125.5) (width 0.2) (layer "F.Cu") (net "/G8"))
 (segment (start 118.5 127.5) (end 120.5 125.5) (width 0.2) (layer "F.Cu") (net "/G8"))
 (segment (start 119.12 101.46) (end 120.5 102.84) (width 0.2) (layer "F.Cu") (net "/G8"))
 (segment (start 80.88 92.42) (end 79.5 93.8) (width 0.2) (layer "B.Cu") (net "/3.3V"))
 (segment (start 103.88 88.76) (end 100.22 92.42) (width 0.2) (layer "B.Cu") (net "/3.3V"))
 (segment (start 100.22 92.42) (end 80.88 92.42) (width 0.2) (layer "B.Cu") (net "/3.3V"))
 (segment (start 79.5 93.8) (end 78 95.3) (width 0.2) (layer "B.Cu") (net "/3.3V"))
 (segment (start 78 107.54) (end 79.5 109.04) (width 0.2) (layer "B.Cu") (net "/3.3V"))
 (segment (start 78 95.3) (end 78 107.54) (width 0.2) (layer "B.Cu") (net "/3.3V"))
 (segment (start 103.88 84.02) (end 105.16 84.02) (width 0.2) (layer "B.Cu") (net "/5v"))
 (segment (start 84.78 83.68) (end 77.5 90.96) (width 0.2) (layer "B.Cu") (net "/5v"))
 (segment (start 121.5 82.18) (end 129.65 90.33) (width 0.2) (layer "B.Cu") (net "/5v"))
 (segment (start 77.5 90.96) (end 77.5 117.5) (width 0.2) (layer "B.Cu") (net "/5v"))
 (segment (start 77.5 117.5) (end 82.92 122.92) (width 0.2) (layer "B.Cu") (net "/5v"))
 (segment (start 129.65 122.615) (end 128.5 123.765) (width 0.2) (layer "B.Cu") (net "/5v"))
 (segment (start 107 82.18) (end 121.5 82.18) (width 0.2) (layer "B.Cu") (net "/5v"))
 (segment (start 103.88 83.68) (end 84.78 83.68) (width 0.2) (layer "B.Cu") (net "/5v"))
 (segment (start 129.65 90.33) (end 129.65 122.615) (width 0.2) (layer "B.Cu") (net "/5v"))
 (segment (start 105.16 84.02) (end 107 82.18) (width 0.2) (layer "B.Cu") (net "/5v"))
 (segment (start 99.52 101.48) (end 103.166 97.834) (width 0.2) (layer "F.Cu") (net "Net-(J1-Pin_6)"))
 (segment (start 103.166 97.834) (end 118.034 97.834) (width 0.2) (layer "F.Cu") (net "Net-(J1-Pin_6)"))
 (segment (start 79.5 103.96) (end 81.98 101.48) (width 0.2) (layer "F.Cu") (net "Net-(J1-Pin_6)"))
 (segment (start 81.98 101.48) (end 82 101.46) (width 0.2) (layer "F.Cu") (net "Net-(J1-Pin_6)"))
 (segment (start 81.98 101.48) (end 99.52 101.48) (width 0.2) (layer "F.Cu") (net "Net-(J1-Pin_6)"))
 (segment (start 118.034 97.834) (end 119.12 98.92) (width 0.2) (layer "F.Cu") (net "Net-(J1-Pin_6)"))
 (segment (start 119.530582 100) (end 120.174 99.356582) (width 0.2) (layer "F.Cu") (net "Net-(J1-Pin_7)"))
 (segment (start 81.934 104.066) (end 99.783418 104.066) (width 0.2) (layer "F.Cu") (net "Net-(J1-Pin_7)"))
 (segment (start 99.783418 104.066) (end 103.849418 100) (width 0.2) (layer "F.Cu") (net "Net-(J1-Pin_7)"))
 (segment (start 103.849418 100) (end 119.530582 100) (width 0.2) (layer "F.Cu") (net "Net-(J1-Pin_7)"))
 (segment (start 120.174 99.356582) (end 120.174 97.434) (width 0.2) (layer "F.Cu") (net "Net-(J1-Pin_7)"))
 (segment (start 79.5 106.5) (end 81.934 104.066) (width 0.2) (layer "F.Cu") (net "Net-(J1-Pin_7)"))
 (segment (start 120.174 97.434) (end 119.12 96.38) (width 0.2) (layer "F.Cu") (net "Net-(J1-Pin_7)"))
 (segment (start 79.5 98.88) (end 83.054 95.326) (width 0.2) (layer "F.Cu") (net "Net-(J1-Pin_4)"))
 (segment (start 83.054 95.326) (end 117.634 95.326) (width 0.2) (layer "F.Cu") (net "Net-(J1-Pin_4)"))
 (segment (start 117.634 95.326) (end 119.12 93.84) (width 0.2) (layer "F.Cu") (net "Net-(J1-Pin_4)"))
 (segment (start 117.634 92.786) (end 119.12 91.3) (width 0.2) (layer "F.Cu") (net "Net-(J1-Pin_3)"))
 (segment (start 83.054 92.786) (end 117.634 92.786) (width 0.2) (layer "F.Cu") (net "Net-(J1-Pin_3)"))
 (segment (start 79.5 96.34) (end 83.054 92.786) (width 0.2) (layer "F.Cu") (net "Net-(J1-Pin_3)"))
 (segment (start 119.556582 94.894) (end 120.174 94.276582) (width 0.2) (layer "F.Cu") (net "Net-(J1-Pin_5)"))
 (segment (start 119.115418 94.894) (end 119.556582 94.894) (width 0.2) (layer "F.Cu") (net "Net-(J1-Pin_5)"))
 (segment (start 83.486 97.434) (end 116.575418 97.434) (width 0.2) (layer "F.Cu") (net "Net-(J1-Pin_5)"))
 (segment (start 79.5 101.42) (end 83.486 97.434) (width 0.2) (layer "F.Cu") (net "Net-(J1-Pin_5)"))
 (segment (start 116.575418 97.434) (end 119.115418 94.894) (width 0.2) (layer "F.Cu") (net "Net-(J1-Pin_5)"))
 (segment (start 120.174 89.814) (end 119.12 88.76) (width 0.2) (layer "F.Cu") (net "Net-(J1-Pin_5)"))
 (segment (start 120.174 94.276582) (end 120.174 89.814) (width 0.2) (layer "F.Cu") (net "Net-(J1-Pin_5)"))
 (segment (start 122.5 133) (end 122.5 87.06) (width 0.2) (layer "F.Cu") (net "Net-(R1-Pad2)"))
 (segment (start 122.5 87.06) (end 119.12 83.68) (width 0.2) (layer "F.Cu") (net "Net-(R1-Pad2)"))
 (segment (start 117.5 138) (end 122.5 133) (width 0.2) (layer "F.Cu") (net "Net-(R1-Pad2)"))
 (segment (start 115.62 138) (end 117.5 138) (width 0.2) (layer "F.Cu") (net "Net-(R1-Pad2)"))
 (segment (start 104.355 134.355) (end 85.776346 134.355) (width 0.2) (layer "F.Cu") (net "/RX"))
 (segment (start 81.725 131.016346) (end 81.725 126.61) (width 0.2) (layer "F.Cu") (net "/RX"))
 (segment (start 83.351346 131.93) (end 82.638654 131.93) (width 0.2) (layer "F.Cu") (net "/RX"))
 (segment (start 81.725 126.61) (end 82.875 125.46) (width 0.2) (layer "F.Cu") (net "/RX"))
 (segment (start 108 138) (end 104.355 134.355) (width 0.2) (layer "F.Cu") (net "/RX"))
 (segment (start 85.776346 134.355) (end 83.351346 131.93) (width 0.2) (layer "F.Cu") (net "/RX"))
 (segment (start 82.638654 131.93) (end 81.725 131.016346) (width 0.2) (layer "F.Cu") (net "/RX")))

